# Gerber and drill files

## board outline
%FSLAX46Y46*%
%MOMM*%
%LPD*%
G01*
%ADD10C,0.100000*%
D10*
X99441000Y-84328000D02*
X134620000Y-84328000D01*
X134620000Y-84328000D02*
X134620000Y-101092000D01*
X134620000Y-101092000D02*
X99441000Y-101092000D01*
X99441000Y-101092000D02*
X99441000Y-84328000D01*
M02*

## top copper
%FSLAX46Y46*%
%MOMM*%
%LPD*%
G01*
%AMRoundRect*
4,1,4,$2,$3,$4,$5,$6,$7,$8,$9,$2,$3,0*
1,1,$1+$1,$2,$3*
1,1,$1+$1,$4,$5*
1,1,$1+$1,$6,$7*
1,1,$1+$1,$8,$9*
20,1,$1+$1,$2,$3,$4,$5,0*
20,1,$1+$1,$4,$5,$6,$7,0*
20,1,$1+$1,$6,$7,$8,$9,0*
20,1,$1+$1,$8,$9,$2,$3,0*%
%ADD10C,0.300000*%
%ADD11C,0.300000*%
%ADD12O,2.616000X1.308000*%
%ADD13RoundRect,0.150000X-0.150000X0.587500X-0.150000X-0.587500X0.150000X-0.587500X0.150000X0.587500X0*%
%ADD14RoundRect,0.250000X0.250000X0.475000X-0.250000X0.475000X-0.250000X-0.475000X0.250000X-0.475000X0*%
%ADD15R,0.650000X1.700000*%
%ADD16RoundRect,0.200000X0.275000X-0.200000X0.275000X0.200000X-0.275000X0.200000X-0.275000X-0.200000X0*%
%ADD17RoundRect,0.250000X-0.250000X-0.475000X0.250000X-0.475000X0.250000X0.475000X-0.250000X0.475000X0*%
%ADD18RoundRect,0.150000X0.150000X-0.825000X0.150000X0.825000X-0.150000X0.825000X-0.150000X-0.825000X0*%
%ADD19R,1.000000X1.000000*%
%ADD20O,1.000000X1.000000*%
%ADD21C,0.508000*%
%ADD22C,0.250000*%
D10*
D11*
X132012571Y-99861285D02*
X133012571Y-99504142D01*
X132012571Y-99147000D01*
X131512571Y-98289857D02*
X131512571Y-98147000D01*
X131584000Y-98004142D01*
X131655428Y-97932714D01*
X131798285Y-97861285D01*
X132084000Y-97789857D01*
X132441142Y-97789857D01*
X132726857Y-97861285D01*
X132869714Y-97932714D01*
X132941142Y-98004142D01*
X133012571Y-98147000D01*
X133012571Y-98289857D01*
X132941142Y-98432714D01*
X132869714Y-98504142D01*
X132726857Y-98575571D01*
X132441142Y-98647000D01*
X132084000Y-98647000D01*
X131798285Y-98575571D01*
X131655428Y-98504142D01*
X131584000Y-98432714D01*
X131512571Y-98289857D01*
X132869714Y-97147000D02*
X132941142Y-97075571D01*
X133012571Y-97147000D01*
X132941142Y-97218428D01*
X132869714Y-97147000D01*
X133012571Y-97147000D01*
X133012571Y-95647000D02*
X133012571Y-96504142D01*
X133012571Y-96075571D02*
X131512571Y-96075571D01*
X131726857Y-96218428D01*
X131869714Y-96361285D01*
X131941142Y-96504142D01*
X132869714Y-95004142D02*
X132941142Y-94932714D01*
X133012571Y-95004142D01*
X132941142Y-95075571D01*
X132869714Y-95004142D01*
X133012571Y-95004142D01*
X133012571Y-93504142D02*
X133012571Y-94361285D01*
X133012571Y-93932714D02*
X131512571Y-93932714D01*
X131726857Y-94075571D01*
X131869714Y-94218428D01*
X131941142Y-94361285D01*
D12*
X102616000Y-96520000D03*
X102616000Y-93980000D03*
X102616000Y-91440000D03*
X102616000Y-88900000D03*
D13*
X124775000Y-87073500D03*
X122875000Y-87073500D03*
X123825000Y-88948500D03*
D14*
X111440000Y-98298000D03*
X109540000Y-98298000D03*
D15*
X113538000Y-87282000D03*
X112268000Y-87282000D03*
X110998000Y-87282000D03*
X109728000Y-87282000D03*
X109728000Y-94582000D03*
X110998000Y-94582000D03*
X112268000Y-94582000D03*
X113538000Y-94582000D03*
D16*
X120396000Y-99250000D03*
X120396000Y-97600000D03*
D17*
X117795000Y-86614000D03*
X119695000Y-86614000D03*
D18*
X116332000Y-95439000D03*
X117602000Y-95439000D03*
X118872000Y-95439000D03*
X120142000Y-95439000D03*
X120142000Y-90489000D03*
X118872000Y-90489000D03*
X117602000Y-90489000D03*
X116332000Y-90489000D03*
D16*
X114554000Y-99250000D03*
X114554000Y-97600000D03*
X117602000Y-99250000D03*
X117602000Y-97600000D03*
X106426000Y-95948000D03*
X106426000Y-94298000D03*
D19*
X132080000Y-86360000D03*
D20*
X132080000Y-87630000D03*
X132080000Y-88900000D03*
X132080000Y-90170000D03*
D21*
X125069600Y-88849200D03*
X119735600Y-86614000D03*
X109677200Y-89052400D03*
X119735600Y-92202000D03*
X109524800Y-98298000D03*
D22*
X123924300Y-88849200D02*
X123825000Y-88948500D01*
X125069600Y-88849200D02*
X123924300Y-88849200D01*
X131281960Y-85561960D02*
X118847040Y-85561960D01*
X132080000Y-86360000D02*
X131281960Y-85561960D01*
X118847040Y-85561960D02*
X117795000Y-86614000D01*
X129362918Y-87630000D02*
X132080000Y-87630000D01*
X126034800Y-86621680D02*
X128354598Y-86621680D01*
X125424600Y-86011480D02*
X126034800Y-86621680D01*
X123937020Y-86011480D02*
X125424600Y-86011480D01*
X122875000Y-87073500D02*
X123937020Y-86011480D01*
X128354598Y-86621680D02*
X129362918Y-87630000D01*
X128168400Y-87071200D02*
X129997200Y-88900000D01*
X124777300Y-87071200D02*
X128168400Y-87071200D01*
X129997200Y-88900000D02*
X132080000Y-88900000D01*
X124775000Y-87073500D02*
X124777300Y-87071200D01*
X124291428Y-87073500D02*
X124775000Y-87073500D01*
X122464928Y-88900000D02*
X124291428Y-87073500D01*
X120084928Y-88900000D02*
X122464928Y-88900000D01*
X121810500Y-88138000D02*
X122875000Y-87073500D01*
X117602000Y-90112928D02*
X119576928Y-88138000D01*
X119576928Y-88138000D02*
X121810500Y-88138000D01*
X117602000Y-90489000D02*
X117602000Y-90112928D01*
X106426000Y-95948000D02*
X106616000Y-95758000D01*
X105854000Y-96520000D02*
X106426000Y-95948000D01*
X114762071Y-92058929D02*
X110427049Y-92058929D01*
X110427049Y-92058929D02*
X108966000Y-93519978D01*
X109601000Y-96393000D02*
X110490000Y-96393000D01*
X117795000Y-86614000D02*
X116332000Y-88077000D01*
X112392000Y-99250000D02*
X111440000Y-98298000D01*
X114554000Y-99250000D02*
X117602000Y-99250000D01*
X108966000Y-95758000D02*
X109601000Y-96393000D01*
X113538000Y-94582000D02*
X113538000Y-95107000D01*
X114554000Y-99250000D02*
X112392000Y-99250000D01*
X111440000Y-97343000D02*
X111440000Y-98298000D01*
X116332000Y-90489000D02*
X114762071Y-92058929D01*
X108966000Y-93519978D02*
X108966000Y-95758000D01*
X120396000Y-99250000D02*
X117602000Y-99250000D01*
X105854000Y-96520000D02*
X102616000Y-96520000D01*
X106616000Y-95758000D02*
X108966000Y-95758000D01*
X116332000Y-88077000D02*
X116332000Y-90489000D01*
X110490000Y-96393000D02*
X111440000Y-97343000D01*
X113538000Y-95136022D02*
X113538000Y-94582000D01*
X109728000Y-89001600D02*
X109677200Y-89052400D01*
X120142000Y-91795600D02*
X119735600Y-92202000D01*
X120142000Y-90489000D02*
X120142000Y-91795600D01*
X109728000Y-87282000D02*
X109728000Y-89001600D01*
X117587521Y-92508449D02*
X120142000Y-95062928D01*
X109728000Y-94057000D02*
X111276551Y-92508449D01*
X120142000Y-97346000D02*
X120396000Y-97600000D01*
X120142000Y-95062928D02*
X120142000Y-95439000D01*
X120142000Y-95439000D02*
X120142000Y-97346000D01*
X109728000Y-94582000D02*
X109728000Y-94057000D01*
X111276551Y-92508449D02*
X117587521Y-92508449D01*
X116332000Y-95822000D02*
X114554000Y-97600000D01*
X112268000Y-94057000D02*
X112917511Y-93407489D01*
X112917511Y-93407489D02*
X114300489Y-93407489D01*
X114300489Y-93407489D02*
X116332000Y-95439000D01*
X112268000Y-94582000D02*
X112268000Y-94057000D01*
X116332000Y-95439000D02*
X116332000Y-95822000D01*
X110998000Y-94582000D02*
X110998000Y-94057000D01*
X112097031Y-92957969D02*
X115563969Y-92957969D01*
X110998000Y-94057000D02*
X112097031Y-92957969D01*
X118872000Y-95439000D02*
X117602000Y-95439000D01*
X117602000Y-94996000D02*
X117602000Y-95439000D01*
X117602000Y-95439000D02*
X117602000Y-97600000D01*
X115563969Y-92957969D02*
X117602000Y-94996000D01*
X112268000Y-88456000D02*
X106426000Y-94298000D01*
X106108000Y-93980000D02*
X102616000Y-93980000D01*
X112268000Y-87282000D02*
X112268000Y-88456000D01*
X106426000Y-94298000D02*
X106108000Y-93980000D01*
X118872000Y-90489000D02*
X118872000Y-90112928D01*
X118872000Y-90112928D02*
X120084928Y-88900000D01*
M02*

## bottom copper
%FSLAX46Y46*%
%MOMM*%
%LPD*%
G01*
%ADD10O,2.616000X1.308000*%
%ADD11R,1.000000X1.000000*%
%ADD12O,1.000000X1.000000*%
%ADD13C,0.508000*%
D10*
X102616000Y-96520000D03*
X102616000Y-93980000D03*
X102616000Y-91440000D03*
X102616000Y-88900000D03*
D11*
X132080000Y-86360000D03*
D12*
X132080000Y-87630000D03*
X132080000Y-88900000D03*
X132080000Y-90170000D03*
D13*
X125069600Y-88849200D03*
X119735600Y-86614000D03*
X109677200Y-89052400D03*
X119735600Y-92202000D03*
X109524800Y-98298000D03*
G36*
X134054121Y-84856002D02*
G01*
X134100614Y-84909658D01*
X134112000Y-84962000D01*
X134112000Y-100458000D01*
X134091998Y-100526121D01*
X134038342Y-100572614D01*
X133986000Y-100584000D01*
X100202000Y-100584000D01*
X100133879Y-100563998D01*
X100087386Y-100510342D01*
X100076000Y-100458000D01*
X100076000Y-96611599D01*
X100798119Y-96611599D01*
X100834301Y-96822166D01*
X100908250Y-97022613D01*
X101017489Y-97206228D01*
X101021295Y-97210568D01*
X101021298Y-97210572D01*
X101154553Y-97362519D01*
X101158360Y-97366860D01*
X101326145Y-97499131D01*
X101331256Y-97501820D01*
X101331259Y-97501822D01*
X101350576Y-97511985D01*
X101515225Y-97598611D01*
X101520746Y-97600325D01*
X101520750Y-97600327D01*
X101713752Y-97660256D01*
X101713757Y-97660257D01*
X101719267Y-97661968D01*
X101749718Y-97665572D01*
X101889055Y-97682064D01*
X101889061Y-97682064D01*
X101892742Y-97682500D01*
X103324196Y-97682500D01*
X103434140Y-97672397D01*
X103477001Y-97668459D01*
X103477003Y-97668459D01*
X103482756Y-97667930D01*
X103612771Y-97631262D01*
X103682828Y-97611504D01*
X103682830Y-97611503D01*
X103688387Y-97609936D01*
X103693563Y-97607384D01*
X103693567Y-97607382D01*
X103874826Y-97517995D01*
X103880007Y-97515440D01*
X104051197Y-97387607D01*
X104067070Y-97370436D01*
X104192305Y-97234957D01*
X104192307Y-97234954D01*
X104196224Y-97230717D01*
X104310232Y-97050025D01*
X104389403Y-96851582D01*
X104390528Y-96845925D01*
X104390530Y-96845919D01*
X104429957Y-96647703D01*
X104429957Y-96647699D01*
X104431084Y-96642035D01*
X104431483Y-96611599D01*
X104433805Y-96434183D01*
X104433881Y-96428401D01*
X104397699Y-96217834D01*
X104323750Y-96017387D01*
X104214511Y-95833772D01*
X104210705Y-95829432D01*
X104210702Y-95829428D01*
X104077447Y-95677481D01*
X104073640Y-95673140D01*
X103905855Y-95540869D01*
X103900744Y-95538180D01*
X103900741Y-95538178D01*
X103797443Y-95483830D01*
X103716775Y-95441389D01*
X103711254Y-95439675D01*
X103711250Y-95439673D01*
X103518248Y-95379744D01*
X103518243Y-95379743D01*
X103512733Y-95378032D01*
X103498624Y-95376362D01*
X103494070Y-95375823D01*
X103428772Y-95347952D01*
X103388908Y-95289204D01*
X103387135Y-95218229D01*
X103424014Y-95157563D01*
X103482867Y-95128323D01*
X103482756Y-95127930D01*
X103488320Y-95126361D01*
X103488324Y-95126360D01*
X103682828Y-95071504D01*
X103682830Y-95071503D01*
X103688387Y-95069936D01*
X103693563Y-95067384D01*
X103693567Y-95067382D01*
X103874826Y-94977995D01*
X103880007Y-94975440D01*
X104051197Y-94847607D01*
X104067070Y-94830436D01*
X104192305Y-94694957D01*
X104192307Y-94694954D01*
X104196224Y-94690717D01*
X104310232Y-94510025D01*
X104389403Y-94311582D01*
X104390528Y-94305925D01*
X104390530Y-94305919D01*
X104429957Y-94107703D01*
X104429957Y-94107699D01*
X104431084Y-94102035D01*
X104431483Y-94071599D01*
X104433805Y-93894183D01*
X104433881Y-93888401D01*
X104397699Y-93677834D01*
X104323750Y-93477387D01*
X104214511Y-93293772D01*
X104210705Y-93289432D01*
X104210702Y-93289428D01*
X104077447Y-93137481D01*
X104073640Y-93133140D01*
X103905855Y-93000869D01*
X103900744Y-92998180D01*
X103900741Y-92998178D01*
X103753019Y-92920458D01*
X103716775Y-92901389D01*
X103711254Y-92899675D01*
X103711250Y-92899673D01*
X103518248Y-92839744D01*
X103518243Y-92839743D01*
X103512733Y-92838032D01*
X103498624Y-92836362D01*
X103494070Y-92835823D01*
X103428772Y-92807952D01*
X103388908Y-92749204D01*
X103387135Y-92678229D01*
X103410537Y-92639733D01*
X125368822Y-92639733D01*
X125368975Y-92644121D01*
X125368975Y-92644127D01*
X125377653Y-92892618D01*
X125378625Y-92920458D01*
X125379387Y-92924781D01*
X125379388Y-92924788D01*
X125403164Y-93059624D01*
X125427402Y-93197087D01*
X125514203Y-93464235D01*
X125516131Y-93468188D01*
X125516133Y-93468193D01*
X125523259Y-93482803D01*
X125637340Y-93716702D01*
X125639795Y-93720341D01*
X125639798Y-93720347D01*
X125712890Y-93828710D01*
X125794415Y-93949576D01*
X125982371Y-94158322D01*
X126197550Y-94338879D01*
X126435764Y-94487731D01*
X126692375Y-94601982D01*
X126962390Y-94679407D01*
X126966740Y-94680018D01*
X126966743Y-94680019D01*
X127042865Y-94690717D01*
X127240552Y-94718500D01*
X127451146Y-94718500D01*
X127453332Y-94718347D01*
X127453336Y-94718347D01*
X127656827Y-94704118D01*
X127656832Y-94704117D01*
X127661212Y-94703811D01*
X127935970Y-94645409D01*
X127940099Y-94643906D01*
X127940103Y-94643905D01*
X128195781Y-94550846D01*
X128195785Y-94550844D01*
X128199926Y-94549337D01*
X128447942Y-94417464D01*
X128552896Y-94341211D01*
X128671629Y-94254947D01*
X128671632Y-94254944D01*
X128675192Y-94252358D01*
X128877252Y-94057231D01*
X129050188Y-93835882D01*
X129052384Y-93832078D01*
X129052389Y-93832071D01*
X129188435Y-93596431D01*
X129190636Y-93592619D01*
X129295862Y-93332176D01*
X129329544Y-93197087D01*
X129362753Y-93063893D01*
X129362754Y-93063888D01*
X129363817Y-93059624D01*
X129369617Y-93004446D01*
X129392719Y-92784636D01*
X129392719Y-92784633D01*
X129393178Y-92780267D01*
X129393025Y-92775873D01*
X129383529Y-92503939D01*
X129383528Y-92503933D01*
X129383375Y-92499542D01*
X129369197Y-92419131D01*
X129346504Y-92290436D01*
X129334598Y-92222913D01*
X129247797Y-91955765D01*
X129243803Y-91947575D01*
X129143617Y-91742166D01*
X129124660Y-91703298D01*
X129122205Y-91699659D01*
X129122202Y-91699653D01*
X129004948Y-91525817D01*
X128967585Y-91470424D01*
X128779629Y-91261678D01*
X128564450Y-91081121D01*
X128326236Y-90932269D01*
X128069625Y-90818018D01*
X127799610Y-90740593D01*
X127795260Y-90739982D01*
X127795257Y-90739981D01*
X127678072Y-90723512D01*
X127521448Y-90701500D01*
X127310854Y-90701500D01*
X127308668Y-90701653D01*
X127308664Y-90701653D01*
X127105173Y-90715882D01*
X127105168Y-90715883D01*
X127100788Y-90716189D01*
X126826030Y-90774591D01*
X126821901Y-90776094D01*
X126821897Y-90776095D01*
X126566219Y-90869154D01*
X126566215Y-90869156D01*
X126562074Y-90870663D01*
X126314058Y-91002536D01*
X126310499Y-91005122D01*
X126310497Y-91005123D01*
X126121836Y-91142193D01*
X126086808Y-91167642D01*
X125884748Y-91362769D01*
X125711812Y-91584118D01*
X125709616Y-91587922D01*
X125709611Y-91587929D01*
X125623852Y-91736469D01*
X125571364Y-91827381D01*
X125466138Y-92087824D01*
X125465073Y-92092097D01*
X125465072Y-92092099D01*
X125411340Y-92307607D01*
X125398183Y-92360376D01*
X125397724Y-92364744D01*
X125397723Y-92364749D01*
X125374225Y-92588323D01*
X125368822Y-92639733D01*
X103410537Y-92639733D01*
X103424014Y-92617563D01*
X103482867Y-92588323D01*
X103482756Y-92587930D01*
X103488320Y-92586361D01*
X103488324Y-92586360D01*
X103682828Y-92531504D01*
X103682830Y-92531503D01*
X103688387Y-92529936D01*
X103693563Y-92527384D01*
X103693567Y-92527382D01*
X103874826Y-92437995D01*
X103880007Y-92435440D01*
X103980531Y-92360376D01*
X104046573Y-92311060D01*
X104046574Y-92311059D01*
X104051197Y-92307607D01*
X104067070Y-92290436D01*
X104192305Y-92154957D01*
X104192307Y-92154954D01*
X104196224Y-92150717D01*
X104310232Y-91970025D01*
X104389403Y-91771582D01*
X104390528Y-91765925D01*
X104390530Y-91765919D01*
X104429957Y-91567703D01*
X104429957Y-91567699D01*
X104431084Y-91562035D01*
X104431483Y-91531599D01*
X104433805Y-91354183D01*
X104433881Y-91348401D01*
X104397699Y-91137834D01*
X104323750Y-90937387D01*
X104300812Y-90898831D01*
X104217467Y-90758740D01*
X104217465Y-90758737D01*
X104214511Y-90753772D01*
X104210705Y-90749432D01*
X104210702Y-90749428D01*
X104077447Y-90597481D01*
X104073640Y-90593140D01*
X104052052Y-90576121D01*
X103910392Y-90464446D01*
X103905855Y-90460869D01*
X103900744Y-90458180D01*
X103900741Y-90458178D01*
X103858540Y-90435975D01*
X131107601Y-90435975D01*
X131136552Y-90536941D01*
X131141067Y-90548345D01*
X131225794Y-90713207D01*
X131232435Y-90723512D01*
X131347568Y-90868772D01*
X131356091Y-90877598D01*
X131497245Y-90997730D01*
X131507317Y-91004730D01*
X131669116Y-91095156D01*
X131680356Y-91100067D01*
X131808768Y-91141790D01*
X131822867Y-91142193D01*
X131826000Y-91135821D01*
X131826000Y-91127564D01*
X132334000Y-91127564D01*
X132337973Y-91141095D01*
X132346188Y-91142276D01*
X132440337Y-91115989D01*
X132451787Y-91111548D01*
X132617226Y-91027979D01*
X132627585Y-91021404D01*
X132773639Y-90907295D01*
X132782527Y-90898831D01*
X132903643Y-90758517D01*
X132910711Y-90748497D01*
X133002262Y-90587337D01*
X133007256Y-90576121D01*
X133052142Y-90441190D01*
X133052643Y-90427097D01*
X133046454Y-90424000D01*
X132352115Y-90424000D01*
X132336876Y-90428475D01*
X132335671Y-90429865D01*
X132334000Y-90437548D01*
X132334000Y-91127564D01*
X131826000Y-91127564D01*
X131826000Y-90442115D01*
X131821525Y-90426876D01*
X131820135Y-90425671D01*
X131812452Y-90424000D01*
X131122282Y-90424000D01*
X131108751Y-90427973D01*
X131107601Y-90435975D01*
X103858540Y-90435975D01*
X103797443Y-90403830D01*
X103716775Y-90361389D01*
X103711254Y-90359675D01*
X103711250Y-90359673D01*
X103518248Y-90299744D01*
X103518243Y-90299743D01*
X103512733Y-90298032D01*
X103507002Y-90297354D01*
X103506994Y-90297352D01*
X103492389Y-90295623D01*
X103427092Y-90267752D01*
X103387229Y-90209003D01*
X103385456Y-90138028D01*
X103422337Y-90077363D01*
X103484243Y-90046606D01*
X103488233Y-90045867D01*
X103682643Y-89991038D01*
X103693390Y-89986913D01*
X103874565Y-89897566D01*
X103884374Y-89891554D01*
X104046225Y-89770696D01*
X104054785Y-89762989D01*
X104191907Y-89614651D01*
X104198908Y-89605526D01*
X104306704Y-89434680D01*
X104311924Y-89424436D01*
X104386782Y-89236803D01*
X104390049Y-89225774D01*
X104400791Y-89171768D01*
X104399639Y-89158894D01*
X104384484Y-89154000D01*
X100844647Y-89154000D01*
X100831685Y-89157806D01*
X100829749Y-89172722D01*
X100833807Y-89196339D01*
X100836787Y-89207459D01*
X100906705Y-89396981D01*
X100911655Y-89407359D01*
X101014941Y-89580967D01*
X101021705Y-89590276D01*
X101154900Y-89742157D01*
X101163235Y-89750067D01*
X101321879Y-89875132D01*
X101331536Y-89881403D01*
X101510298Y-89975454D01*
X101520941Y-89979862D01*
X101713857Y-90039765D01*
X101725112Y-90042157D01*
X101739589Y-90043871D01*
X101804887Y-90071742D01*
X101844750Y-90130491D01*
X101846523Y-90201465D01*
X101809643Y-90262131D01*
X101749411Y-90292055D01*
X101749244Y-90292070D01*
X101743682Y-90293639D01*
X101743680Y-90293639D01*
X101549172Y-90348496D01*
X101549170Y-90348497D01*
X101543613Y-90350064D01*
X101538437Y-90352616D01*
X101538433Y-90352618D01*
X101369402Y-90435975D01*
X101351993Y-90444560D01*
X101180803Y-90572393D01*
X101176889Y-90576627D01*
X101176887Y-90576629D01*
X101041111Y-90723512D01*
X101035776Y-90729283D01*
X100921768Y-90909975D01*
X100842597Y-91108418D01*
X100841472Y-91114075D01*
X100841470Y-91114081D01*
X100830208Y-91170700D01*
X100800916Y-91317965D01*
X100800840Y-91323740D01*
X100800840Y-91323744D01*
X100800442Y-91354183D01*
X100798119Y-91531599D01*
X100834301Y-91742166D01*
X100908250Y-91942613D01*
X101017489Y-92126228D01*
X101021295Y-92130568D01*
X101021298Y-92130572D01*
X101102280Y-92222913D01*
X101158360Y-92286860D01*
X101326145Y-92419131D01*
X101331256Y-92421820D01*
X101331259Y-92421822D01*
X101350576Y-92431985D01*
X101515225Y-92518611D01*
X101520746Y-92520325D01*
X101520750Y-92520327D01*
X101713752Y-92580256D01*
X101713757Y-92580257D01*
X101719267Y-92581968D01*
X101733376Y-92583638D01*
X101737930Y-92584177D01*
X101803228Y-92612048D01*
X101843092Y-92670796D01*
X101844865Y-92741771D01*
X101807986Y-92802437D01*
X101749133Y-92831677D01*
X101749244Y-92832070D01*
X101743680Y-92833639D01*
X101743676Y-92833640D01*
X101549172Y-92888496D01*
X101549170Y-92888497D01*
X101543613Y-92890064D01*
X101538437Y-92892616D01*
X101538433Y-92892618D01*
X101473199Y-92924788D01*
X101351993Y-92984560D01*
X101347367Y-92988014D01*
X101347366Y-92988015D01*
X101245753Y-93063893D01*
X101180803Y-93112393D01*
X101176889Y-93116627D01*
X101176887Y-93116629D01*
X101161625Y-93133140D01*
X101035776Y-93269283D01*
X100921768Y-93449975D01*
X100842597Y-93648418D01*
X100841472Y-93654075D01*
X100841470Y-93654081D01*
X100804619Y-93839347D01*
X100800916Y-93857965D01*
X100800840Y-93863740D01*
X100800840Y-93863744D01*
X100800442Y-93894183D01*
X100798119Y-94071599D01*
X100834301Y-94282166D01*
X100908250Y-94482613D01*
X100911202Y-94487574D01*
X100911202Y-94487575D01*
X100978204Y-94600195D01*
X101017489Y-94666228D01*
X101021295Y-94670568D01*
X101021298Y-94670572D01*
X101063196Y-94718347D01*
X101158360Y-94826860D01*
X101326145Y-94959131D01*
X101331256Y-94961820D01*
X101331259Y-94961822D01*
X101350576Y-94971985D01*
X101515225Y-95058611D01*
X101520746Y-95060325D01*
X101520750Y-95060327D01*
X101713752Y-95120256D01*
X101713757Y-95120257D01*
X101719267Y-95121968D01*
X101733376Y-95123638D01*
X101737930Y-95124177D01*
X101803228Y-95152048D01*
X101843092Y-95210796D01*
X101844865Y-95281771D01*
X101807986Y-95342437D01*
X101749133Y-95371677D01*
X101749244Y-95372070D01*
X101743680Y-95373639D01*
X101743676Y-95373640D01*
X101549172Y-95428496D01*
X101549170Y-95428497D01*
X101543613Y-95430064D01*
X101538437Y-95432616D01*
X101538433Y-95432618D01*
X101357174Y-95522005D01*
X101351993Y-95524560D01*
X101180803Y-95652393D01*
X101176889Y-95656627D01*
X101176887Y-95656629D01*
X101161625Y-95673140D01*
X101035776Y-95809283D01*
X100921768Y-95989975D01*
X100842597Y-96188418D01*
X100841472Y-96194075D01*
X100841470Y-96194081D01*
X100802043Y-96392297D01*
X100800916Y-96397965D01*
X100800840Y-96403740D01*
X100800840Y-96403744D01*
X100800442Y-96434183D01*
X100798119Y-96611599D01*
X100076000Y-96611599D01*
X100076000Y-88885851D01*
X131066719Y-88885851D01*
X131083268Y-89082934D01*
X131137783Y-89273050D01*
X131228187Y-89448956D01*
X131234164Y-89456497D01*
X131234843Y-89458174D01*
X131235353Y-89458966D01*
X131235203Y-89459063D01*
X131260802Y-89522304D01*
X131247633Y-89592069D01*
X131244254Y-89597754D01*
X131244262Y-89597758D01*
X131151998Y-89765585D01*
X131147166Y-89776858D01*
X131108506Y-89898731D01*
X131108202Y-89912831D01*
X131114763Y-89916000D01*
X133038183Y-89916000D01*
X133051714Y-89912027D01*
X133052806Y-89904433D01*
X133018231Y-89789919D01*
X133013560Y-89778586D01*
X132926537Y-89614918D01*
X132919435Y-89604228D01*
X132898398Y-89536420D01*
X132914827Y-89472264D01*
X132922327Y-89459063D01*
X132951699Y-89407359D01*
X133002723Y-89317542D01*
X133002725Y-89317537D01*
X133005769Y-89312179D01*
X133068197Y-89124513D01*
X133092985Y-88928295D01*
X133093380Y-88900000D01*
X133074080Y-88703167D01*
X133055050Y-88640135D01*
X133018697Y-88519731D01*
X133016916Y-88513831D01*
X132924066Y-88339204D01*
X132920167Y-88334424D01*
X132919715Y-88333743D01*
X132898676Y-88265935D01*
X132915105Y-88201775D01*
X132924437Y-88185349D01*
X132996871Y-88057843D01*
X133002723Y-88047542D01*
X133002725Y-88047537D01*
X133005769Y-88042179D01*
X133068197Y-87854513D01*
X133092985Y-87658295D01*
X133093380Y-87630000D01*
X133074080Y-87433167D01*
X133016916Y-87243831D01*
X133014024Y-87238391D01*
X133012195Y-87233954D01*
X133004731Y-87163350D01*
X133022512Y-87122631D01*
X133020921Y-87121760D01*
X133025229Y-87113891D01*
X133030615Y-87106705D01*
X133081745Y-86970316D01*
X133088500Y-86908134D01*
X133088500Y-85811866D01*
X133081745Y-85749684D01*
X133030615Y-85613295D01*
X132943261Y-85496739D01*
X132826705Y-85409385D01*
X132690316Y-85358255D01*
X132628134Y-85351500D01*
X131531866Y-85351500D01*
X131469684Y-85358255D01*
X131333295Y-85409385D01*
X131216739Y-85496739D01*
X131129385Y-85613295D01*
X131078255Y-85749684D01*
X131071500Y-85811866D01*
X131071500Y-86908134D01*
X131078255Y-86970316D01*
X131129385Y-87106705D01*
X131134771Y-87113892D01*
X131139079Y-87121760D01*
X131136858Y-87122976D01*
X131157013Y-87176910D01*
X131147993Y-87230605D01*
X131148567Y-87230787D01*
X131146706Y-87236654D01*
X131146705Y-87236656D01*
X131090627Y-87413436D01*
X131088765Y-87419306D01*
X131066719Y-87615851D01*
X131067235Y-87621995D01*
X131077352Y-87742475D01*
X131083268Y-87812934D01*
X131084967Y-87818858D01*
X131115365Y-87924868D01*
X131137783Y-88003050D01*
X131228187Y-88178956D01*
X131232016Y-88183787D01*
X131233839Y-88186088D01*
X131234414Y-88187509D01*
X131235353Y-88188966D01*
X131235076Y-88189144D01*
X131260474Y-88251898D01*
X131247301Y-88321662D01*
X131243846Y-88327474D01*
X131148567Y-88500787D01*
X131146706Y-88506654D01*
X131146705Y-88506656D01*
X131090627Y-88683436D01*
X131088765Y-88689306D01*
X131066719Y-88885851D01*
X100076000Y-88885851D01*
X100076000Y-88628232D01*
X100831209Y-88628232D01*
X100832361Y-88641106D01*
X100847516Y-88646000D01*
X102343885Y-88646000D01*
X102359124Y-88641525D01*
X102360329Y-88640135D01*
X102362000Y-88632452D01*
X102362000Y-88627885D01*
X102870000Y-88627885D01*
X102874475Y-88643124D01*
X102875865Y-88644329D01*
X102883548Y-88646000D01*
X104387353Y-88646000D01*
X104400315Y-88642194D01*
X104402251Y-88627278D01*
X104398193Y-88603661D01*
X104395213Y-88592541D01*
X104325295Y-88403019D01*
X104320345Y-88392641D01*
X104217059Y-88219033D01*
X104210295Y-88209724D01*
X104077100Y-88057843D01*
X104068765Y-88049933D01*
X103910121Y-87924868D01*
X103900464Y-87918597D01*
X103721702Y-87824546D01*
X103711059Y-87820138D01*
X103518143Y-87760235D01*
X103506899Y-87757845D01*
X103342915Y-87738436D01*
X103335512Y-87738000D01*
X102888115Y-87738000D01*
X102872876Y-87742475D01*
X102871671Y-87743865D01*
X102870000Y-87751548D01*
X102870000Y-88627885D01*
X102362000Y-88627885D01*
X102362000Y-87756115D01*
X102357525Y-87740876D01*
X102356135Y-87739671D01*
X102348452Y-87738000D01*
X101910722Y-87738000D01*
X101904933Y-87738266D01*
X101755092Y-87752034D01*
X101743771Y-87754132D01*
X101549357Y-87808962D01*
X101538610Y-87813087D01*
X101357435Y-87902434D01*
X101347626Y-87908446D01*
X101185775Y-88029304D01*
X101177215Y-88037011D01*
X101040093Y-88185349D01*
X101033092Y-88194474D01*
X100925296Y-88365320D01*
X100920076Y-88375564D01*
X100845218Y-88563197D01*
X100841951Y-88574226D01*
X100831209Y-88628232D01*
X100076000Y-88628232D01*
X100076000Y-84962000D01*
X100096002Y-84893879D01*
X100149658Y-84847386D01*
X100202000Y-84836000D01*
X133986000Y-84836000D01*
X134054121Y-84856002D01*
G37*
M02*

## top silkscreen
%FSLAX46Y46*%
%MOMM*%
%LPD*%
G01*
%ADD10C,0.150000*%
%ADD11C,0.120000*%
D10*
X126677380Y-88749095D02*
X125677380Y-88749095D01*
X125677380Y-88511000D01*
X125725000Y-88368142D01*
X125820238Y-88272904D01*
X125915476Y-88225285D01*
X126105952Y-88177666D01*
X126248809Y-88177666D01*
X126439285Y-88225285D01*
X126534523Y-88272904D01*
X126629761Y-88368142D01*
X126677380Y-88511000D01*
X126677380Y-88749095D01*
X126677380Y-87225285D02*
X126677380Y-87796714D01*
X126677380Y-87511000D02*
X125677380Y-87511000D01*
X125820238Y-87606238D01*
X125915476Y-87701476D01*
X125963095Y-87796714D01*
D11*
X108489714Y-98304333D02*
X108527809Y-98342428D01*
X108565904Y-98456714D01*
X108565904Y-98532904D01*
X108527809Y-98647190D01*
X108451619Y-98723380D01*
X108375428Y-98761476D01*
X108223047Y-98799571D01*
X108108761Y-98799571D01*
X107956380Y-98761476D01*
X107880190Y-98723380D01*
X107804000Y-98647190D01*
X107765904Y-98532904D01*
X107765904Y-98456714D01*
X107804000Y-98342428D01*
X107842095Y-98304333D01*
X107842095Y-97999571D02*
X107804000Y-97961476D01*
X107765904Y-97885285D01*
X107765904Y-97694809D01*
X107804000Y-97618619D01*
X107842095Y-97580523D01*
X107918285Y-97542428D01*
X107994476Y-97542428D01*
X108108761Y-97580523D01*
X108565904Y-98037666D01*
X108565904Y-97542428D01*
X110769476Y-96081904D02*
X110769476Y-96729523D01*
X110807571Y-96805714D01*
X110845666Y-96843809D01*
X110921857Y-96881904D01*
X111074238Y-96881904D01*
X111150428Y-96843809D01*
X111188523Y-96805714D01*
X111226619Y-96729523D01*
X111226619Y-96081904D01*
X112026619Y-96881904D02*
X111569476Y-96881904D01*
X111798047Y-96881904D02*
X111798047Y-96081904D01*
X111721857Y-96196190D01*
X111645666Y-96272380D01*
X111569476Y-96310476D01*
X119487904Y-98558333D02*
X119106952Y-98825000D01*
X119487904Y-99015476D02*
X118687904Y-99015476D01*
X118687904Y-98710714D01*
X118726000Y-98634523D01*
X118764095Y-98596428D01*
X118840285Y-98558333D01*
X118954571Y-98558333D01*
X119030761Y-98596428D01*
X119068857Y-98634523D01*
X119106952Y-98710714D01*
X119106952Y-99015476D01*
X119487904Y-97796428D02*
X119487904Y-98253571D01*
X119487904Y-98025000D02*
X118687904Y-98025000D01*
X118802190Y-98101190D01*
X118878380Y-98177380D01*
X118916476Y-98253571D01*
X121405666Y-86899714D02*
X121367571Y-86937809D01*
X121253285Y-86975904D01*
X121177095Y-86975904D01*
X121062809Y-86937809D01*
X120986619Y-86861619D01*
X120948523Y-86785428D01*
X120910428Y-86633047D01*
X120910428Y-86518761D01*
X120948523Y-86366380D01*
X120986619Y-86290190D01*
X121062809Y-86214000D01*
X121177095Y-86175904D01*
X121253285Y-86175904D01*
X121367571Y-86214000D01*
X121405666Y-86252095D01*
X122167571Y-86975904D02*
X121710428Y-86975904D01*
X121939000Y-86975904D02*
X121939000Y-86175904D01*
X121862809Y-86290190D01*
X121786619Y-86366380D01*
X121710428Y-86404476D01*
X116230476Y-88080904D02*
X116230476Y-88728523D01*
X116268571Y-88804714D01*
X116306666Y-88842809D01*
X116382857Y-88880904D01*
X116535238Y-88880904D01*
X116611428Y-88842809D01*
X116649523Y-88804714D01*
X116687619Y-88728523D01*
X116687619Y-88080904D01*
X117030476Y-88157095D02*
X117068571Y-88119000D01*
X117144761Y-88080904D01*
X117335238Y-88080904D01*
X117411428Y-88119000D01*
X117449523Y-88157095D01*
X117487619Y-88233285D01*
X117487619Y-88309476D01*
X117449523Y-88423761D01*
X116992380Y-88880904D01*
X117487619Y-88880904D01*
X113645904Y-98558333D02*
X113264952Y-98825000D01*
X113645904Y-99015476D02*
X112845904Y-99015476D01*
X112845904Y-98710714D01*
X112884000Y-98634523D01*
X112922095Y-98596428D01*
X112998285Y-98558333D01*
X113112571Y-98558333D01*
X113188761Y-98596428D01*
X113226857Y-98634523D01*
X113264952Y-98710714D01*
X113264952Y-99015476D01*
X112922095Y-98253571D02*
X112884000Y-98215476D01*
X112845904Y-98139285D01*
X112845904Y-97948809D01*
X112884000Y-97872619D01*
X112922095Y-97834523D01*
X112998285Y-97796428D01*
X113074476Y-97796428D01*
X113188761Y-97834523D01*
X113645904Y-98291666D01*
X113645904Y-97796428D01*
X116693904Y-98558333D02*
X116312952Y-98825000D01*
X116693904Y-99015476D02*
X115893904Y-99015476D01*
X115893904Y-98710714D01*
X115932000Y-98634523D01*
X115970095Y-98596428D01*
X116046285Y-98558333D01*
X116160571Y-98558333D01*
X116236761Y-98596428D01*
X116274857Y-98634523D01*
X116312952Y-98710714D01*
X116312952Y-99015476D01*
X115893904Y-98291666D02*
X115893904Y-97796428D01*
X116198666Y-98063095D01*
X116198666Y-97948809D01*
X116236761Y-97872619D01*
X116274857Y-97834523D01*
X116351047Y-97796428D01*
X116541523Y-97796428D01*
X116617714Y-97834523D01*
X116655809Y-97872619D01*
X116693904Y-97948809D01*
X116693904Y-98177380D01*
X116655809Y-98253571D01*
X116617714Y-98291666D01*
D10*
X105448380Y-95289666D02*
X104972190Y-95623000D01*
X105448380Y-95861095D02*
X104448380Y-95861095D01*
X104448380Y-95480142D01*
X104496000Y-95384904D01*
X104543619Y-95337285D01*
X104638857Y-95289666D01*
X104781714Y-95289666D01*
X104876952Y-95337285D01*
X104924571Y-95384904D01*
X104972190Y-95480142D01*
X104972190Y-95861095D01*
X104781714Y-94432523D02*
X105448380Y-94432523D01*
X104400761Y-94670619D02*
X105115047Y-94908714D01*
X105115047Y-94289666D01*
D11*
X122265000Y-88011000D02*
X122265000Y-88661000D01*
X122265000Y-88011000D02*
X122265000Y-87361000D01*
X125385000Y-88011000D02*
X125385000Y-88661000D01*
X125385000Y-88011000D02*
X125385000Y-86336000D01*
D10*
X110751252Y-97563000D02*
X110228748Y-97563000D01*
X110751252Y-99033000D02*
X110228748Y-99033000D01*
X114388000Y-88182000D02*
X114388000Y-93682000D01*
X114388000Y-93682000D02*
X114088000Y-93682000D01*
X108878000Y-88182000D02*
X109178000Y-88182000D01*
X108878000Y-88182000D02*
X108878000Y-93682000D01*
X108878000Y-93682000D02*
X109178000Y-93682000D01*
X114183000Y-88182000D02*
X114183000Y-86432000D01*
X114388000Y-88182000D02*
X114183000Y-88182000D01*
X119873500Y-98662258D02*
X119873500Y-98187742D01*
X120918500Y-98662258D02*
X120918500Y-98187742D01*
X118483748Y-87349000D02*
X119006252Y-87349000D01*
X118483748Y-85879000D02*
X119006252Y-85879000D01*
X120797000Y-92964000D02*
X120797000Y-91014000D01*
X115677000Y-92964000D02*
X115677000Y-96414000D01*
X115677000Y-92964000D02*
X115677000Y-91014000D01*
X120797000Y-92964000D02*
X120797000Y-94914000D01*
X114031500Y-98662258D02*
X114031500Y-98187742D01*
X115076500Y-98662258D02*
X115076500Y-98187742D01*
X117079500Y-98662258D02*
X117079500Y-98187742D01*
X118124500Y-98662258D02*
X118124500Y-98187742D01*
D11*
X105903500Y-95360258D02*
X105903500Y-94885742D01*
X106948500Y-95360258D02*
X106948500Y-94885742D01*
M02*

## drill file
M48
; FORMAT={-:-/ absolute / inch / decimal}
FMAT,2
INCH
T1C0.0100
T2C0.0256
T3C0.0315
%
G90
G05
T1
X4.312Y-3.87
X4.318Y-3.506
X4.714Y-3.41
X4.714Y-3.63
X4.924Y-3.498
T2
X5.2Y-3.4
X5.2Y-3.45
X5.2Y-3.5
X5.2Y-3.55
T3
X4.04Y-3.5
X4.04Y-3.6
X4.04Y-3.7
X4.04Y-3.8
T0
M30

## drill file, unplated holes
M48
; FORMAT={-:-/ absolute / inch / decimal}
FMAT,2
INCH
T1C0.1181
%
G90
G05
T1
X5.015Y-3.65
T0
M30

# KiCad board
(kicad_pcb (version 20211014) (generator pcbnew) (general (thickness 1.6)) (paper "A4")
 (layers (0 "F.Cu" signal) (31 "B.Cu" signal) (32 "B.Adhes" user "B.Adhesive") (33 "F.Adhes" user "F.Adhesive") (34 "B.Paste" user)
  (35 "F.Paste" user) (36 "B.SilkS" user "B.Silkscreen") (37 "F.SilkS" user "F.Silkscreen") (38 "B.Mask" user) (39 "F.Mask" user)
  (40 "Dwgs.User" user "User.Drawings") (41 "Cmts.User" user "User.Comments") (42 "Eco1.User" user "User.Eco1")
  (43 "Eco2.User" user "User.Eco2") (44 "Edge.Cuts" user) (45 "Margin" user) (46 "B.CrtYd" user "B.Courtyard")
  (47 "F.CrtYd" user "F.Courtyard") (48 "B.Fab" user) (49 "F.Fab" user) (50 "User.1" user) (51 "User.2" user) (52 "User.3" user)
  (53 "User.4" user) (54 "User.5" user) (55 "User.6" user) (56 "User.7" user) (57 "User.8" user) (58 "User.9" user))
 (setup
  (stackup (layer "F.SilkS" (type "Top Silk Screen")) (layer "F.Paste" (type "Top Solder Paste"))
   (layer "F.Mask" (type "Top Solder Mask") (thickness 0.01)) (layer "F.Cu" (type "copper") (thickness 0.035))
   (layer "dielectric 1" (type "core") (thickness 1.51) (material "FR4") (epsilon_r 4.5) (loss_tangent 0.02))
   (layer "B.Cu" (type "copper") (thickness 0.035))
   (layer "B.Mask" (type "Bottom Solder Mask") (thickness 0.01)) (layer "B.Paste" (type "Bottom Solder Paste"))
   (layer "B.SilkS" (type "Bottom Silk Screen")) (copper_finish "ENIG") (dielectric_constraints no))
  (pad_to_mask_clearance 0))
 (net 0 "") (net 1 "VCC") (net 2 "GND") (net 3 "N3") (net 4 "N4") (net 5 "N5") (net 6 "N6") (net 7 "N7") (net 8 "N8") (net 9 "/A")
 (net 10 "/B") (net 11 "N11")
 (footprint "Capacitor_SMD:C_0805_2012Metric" (layer "F.Cu") (at 110.49 98.298 180)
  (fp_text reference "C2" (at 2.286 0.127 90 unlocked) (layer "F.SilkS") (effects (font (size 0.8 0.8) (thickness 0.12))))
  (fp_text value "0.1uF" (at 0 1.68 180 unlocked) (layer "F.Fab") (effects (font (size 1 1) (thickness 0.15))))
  (fp_line (start -0.261252 0.735) (end 0.261252 0.735) (layer "F.SilkS") (width 0.15))
  (fp_line (start -0.261252 -0.735) (end 0.261252 -0.735) (layer "F.SilkS") (width 0.15))
  (pad "1" smd roundrect locked (at -0.95 0 180) (size 1 1.45) (layers "F.Cu" "F.Paste" "F.Mask") (roundrect_rratio 0.25) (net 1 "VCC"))
  (pad "2" smd roundrect locked (at 0.95 0 180) (size 1 1.45) (layers "F.Cu" "F.Paste" "F.Mask") (roundrect_rratio 0.25) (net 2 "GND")))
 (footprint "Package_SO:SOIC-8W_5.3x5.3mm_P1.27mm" (layer "F.Cu") (at 111.633 90.932 -90)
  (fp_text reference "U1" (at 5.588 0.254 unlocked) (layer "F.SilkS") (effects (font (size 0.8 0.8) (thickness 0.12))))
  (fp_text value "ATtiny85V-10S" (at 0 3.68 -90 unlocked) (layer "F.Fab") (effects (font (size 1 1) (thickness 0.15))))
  (fp_line (start -2.75 -2.755) (end 2.75 -2.755) (layer "F.SilkS") (width 0.15))
  (fp_line (start 2.75 -2.755) (end 2.75 -2.455) (layer "F.SilkS") (width 0.15))
  (fp_line (start -2.75 2.755) (end -2.75 2.455) (layer "F.SilkS") (width 0.15))
  (fp_line (start -2.75 2.755) (end 2.75 2.755) (layer "F.SilkS") (width 0.15))
  (fp_line (start 2.75 2.755) (end 2.75 2.455) (layer "F.SilkS") (width 0.15))
  (fp_line (start -2.75 -2.55) (end -4.5 -2.55) (layer "F.SilkS") (width 0.15))
  (fp_line (start -2.75 -2.755) (end -2.75 -2.55) (layer "F.SilkS") (width 0.15))
  (pad "1" smd rect locked (at -3.65 -1.905 270) (size 1.7 0.65) (layers "F.Cu" "F.Paste" "F.Mask") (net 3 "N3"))
  (pad "2" smd rect locked (at -3.65 -0.635 270) (size 1.7 0.65) (layers "F.Cu" "F.Paste" "F.Mask") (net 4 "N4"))
  (pad "3" smd rect locked (at -3.65 0.635 270) (size 1.7 0.65) (layers "F.Cu" "F.Paste" "F.Mask") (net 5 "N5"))
  (pad "4" smd rect locked (at -3.65 1.905 270) (size 1.7 0.65) (layers "F.Cu" "F.Paste" "F.Mask") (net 2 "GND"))
  (pad "5" smd rect locked (at 3.65 1.905 270) (size 1.7 0.65) (layers "F.Cu" "F.Paste" "F.Mask") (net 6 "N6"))
  (pad "6" smd rect locked (at 3.65 0.635 270) (size 1.7 0.65) (layers "F.Cu" "F.Paste" "F.Mask") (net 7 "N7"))
  (pad "7" smd rect locked (at 3.65 -0.635 270) (size 1.7 0.65) (layers "F.Cu" "F.Paste" "F.Mask") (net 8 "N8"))
  (pad "8" smd rect locked (at 3.65 -1.905 270) (size 1.7 0.65) (layers "F.Cu" "F.Paste" "F.Mask") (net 1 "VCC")))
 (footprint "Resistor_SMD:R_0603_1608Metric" (layer "F.Cu") (at 120.396 98.425 90)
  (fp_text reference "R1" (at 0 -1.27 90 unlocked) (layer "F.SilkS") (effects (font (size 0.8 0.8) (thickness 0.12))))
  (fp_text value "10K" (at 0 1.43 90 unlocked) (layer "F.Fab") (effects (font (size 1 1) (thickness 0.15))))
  (fp_line (start -0.237258 -0.5225) (end 0.237258 -0.5225) (layer "F.SilkS") (width 0.15))
  (fp_line (start -0.237258 0.5225) (end 0.237258 0.5225) (layer "F.SilkS") (width 0.15))
  (pad "1" smd roundrect locked (at -0.825 0 90) (size 0.8 0.95) (layers "F.Cu" "F.Paste" "F.Mask") (roundrect_rratio 0.25) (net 1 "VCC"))
  (pad "2" smd roundrect locked (at 0.825 0 90) (size 0.8 0.95) (layers "F.Cu" "F.Paste" "F.Mask") (roundrect_rratio 0.25) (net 6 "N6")))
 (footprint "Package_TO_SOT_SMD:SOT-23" (layer "F.Cu") (at 123.825 88.011 -90)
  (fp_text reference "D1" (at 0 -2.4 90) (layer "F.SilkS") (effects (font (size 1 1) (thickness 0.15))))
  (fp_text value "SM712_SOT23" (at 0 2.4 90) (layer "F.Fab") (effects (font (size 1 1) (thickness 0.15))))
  (fp_line (start 0 -1.56) (end -1.675 -1.56) (layer "F.SilkS") (width 0.12))
  (fp_line (start 0 1.56) (end 0.65 1.56) (layer "F.SilkS") (width 0.12))
  (fp_line (start 0 -1.56) (end 0.65 -1.56) (layer "F.SilkS") (width 0.12))
  (fp_line (start 0 1.56) (end -0.65 1.56) (layer "F.SilkS") (width 0.12))
  (pad "1" smd roundrect locked (at -0.9375 -0.95 270) (size 1.475 0.6) (layers "F.Cu" "F.Paste" "F.Mask") (roundrect_rratio 0.25)
   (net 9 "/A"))
  (pad "2" smd roundrect locked (at -0.9375 0.95 270) (size 1.475 0.6) (layers "F.Cu" "F.Paste" "F.Mask") (roundrect_rratio 0.25)
   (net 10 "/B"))
  (pad "3" smd roundrect locked (at 0.9375 0 270) (size 1.475 0.6) (layers "F.Cu" "F.Paste" "F.Mask") (roundrect_rratio 0.25) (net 2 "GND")))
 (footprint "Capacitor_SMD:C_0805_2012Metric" (layer "F.Cu") (at 118.745 86.614)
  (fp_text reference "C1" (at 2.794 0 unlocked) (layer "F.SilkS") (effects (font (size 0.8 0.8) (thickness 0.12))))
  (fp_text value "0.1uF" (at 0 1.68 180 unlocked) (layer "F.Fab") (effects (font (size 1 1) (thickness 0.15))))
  (fp_line (start -0.261252 0.735) (end 0.261252 0.735) (layer "F.SilkS") (width 0.15))
  (fp_line (start -0.261252 -0.735) (end 0.261252 -0.735) (layer "F.SilkS") (width 0.15))
  (pad "1" smd roundrect locked (at -0.95 0) (size 1 1.45) (layers "F.Cu" "F.Paste" "F.Mask") (roundrect_rratio 0.25) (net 1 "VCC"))
  (pad "2" smd roundrect locked (at 0.95 0) (size 1 1.45) (layers "F.Cu" "F.Paste" "F.Mask") (roundrect_rratio 0.25) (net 2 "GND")))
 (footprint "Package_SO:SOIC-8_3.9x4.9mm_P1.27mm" (layer "F.Cu") (at 118.237 92.964 90)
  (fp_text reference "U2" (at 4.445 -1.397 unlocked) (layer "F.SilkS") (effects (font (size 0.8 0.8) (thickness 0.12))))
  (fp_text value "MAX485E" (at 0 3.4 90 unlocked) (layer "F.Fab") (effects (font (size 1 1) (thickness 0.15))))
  (fp_line (start 0 2.56) (end 1.95 2.56) (layer "F.SilkS") (width 0.15))
  (fp_line (start 0 -2.56) (end -3.45 -2.56) (layer "F.SilkS") (width 0.15))
  (fp_line (start 0 -2.56) (end 1.95 -2.56) (layer "F.SilkS") (width 0.15))
  (fp_line (start 0 2.56) (end -1.95 2.56) (layer "F.SilkS") (width 0.15))
  (pad "1" smd roundrect locked (at -2.475 -1.905 90) (size 1.95 0.6) (layers "F.Cu" "F.Paste" "F.Mask") (roundrect_rratio 0.25)
   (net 8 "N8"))
  (pad "2" smd roundrect locked (at -2.475 -0.635 90) (size 1.95 0.6) (layers "F.Cu" "F.Paste" "F.Mask") (roundrect_rratio 0.25)
   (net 7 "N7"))
  (pad "3" smd roundrect locked (at -2.475 0.635 90) (size 1.95 0.6) (layers "F.Cu" "F.Paste" "F.Mask") (roundrect_rratio 0.25) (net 7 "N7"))
  (pad "4" smd roundrect locked (at -2.475 1.905 90) (size 1.95 0.6) (layers "F.Cu" "F.Paste" "F.Mask") (roundrect_rratio 0.25) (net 6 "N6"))
  (pad "5" smd roundrect locked (at 2.475 1.905 90) (size 1.95 0.6) (layers "F.Cu" "F.Paste" "F.Mask") (roundrect_rratio 0.25) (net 2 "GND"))
  (pad "6" smd roundrect locked (at 2.475 0.635 90) (size 1.95 0.6) (layers "F.Cu" "F.Paste" "F.Mask") (roundrect_rratio 0.25) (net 9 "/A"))
  (pad "7" smd roundrect locked (at 2.475 -0.635 90) (size 1.95 0.6) (layers "F.Cu" "F.Paste" "F.Mask") (roundrect_rratio 0.25)
   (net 10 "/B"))
  (pad "8" smd roundrect locked (at 2.475 -1.905 90) (size 1.95 0.6) (layers "F.Cu" "F.Paste" "F.Mask") (roundrect_rratio 0.25)
   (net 1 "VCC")))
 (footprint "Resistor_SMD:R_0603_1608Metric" (layer "F.Cu") (at 114.554 98.425 90)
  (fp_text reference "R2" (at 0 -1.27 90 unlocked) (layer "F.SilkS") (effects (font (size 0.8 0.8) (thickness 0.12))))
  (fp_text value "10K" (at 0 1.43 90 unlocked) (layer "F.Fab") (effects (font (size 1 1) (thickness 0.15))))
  (fp_line (start -0.237258 -0.5225) (end 0.237258 -0.5225) (layer "F.SilkS") (width 0.15))
  (fp_line (start -0.237258 0.5225) (end 0.237258 0.5225) (layer "F.SilkS") (width 0.15))
  (pad "1" smd roundrect locked (at -0.825 0 90) (size 0.8 0.95) (layers "F.Cu" "F.Paste" "F.Mask") (roundrect_rratio 0.25) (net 1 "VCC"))
  (pad "2" smd roundrect locked (at 0.825 0 90) (size 0.8 0.95) (layers "F.Cu" "F.Paste" "F.Mask") (roundrect_rratio 0.25) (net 8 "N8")))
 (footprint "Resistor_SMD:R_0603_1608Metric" (layer "F.Cu") (at 117.602 98.425 90)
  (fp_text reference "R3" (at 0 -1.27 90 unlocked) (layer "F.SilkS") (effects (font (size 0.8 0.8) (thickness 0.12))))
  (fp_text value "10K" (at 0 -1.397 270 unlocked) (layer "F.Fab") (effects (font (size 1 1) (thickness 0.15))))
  (fp_line (start -0.237258 -0.5225) (end 0.237258 -0.5225) (layer "F.SilkS") (width 0.15))
  (fp_line (start -0.237258 0.5225) (end 0.237258 0.5225) (layer "F.SilkS") (width 0.15))
  (pad "1" smd roundrect locked (at -0.825 0 90) (size 0.8 0.95) (layers "F.Cu" "F.Paste" "F.Mask") (roundrect_rratio 0.25) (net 1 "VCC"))
  (pad "2" smd roundrect locked (at 0.825 0 90) (size 0.8 0.95) (layers "F.Cu" "F.Paste" "F.Mask") (roundrect_rratio 0.25) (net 7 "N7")))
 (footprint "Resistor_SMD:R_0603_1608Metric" (layer "F.Cu") (at 106.426 95.123 90)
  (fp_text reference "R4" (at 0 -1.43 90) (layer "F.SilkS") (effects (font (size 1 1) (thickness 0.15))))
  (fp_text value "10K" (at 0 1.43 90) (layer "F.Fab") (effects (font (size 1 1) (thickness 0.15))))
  (fp_line (start -0.237258 -0.5225) (end 0.237258 -0.5225) (layer "F.SilkS") (width 0.12))
  (fp_line (start -0.237258 0.5225) (end 0.237258 0.5225) (layer "F.SilkS") (width 0.12))
  (pad "1" smd roundrect locked (at -0.825 0 90) (size 0.8 0.95) (layers "F.Cu" "F.Paste" "F.Mask") (roundrect_rratio 0.25) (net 1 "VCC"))
  (pad "2" smd roundrect locked (at 0.825 0 90) (size 0.8 0.95) (layers "F.Cu" "F.Paste" "F.Mask") (roundrect_rratio 0.25) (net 4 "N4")))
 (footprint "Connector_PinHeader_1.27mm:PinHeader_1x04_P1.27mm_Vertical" (layer "B.Cu") (at 132.08 86.36 180)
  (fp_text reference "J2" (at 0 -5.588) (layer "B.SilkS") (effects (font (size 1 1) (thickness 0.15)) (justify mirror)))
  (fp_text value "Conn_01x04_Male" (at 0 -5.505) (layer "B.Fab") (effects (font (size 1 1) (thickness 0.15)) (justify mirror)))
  (pad "1" thru_hole rect locked (at 0 0 180) (size 1 1) (drill 0.65) (layers *.Cu *.Mask) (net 1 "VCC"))
  (pad "2" thru_hole oval locked (at 0 -1.27 180) (size 1 1) (drill 0.65) (layers *.Cu *.Mask) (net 10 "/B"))
  (pad "3" thru_hole oval locked (at 0 -2.54 180) (size 1 1) (drill 0.65) (layers *.Cu *.Mask) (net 9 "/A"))
  (pad "4" thru_hole oval locked (at 0 -3.81 180) (size 1 1) (drill 0.65) (layers *.Cu *.Mask) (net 2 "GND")))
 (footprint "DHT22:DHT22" (layer "B.Cu") (at 102.616 92.71 90)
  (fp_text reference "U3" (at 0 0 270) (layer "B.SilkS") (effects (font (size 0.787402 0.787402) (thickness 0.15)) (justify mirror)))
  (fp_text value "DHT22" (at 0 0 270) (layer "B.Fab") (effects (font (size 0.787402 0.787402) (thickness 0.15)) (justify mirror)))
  (pad "" np_thru_hole circle locked (at 0 24.765 90) (size 3 3) (drill 3) (layers *.Cu *.Mask))
  (pad "DATA" thru_hole oval locked (at -1.27 0 90) (size 1.308 2.616) (drill 0.8) (layers *.Cu *.Mask) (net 4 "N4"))
  (pad "GND" thru_hole oval locked (at 3.81 0 90) (size 1.308 2.616) (drill 0.8) (layers *.Cu *.Mask) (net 2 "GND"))
  (pad "NC" thru_hole oval locked (at 1.27 0 90) (size 1.308 2.616) (drill 0.8) (layers *.Cu *.Mask) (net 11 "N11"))
  (pad "VDD" thru_hole oval locked (at -3.81 0 90) (size 1.308 2.616) (drill 0.8) (layers *.Cu *.Mask) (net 1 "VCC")))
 (gr_rect (start 99.441 84.328) (end 134.62 101.092) (layer "Edge.Cuts") (width 0.1) (fill none))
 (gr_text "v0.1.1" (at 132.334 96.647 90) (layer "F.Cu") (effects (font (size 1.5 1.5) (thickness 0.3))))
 (segment (start 106.426 95.948) (end 106.616 95.758) (width 0.25) (layer "F.Cu") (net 1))
 (segment (start 105.854 96.52) (end 106.426 95.948) (width 0.25) (layer "F.Cu") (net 1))
 (segment (start 114.762071 92.058929) (end 110.427049 92.058929) (width 0.25) (layer "F.Cu") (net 1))
 (segment (start 110.427049 92.058929) (end 108.966 93.519978) (width 0.25) (layer "F.Cu") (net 1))
 (segment (start 109.601 96.393) (end 110.49 96.393) (width 0.25) (layer "F.Cu") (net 1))
 (segment (start 117.795 86.614) (end 116.332 88.077) (width 0.25) (layer "F.Cu") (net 1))
 (segment (start 131.28196 85.56196) (end 118.84704 85.56196) (width 0.25) (layer "F.Cu") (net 1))
 (segment (start 112.392 99.25) (end 111.44 98.298) (width 0.25) (layer "F.Cu") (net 1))
 (segment (start 114.554 99.25) (end 117.602 99.25) (width 0.25) (layer "F.Cu") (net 1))
 (segment (start 108.966 95.758) (end 109.601 96.393) (width 0.25) (layer "F.Cu") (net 1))
 (segment (start 113.538 94.582) (end 113.538 95.107) (width 0.25) (layer "F.Cu") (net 1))
 (segment (start 114.554 99.25) (end 112.392 99.25) (width 0.25) (layer "F.Cu") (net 1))
 (segment (start 111.44 97.343) (end 111.44 98.298) (width 0.25) (layer "F.Cu") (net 1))
 (segment (start 116.332 90.489) (end 114.762071 92.058929) (width 0.25) (layer "F.Cu") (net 1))
 (segment (start 108.966 93.519978) (end 108.966 95.758) (width 0.25) (layer "F.Cu") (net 1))
 (segment (start 120.396 99.25) (end 117.602 99.25) (width 0.25) (layer "F.Cu") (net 1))
 (segment (start 105.854 96.52) (end 102.616 96.52) (width 0.25) (layer "F.Cu") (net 1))
 (segment (start 106.616 95.758) (end 108.966 95.758) (width 0.25) (layer "F.Cu") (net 1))
 (segment (start 118.84704 85.56196) (end 117.795 86.614) (width 0.25) (layer "F.Cu") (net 1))
 (segment (start 116.332 88.077) (end 116.332 90.489) (width 0.25) (layer "F.Cu") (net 1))
 (segment (start 110.49 96.393) (end 111.44 97.343) (width 0.25) (layer "F.Cu") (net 1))
 (segment (start 113.538 95.136022) (end 113.538 94.582) (width 0.25) (layer "F.Cu") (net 1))
 (segment (start 132.08 86.36) (end 131.28196 85.56196) (width 0.25) (layer "F.Cu") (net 1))
 (segment (start 109.728 89.0016) (end 109.6772 89.0524) (width 0.25) (layer "F.Cu") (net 2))
 (segment (start 123.9243 88.8492) (end 123.825 88.9485) (width 0.25) (layer "F.Cu") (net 2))
 (segment (start 120.142 91.7956) (end 119.7356 92.202) (width 0.25) (layer "F.Cu") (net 2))
 (segment (start 120.142 90.489) (end 120.142 91.7956) (width 0.25) (layer "F.Cu") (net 2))
 (segment (start 125.0696 88.8492) (end 123.9243 88.8492) (width 0.25) (layer "F.Cu") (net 2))
 (segment (start 109.728 87.282) (end 109.728 89.0016) (width 0.25) (layer "F.Cu") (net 2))
 (via (at 119.7356 86.614) (size 0.508) (drill 0.254) (layers "F.Cu" "B.Cu") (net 2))
 (via (at 109.6772 89.0524) (size 0.508) (drill 0.254) (layers "F.Cu" "B.Cu") (free) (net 2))
 (via (at 119.7356 92.202) (size 0.508) (drill 0.254) (layers "F.Cu" "B.Cu") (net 2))
 (via (at 125.0696 88.8492) (size 0.508) (drill 0.254) (layers "F.Cu" "B.Cu") (free) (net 2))
 (via (at 109.5248 98.298) (size 0.508) (drill 0.254) (layers "F.Cu" "B.Cu") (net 2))
 (segment (start 117.587521 92.508449) (end 120.142 95.062928) (width 0.25) (layer "F.Cu") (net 6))
 (segment (start 109.728 94.057) (end 111.276551 92.508449) (width 0.25) (layer "F.Cu") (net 6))
 (segment (start 120.142 97.346) (end 120.396 97.6) (width 0.25) (layer "F.Cu") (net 6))
 (segment (start 120.142 95.062928) (end 120.142 95.439) (width 0.25) (layer "F.Cu") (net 6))
 (segment (start 120.142 95.439) (end 120.142 97.346) (width 0.25) (layer "F.Cu") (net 6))
 (segment (start 109.728 94.582) (end 109.728 94.057) (width 0.25) (layer "F.Cu") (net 6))
 (segment (start 111.276551 92.508449) (end 117.587521 92.508449) (width 0.25) (layer "F.Cu") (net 6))
 (segment (start 116.332 95.822) (end 114.554 97.6) (width 0.25) (layer "F.Cu") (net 8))
 (segment (start 112.268 94.057) (end 112.917511 93.407489) (width 0.25) (layer "F.Cu") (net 8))
 (segment (start 112.917511 93.407489) (end 114.300489 93.407489) (width 0.25) (layer "F.Cu") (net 8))
 (segment (start 114.300489 93.407489) (end 116.332 95.439) (width 0.25) (layer "F.Cu") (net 8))
 (segment (start 112.268 94.582) (end 112.268 94.057) (width 0.25) (layer "F.Cu") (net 8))
 (segment (start 116.332 95.439) (end 116.332 95.822) (width 0.25) (layer "F.Cu") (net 8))
 (segment (start 110.998 94.582) (end 110.998 94.057) (width 0.25) (layer "F.Cu") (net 7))
 (segment (start 112.097031 92.957969) (end 115.563969 92.957969) (width 0.25) (layer "F.Cu") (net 7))
 (segment (start 110.998 94.057) (end 112.097031 92.957969) (width 0.25) (layer "F.Cu") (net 7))
 (segment (start 118.872 95.439) (end 117.602 95.439) (width 0.25) (layer "F.Cu") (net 7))
 (segment (start 117.602 94.996) (end 117.602 95.439) (width 0.25) (layer "F.Cu") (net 7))
 (segment (start 117.602 95.439) (end 117.602 97.6) (width 0.25) (layer "F.Cu") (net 7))
 (segment (start 115.563969 92.957969) (end 117.602 94.996) (width 0.25) (layer "F.Cu") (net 7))
 (segment (start 129.9972 88.9) (end 132.08 88.9) (width 0.25) (layer "F.Cu") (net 9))
 (segment (start 124.291428 87.0735) (end 124.775 87.0735) (width 0.25) (layer "F.Cu") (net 9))
 (segment (start 128.1684 87.0712) (end 129.9972 88.9) (width 0.25) (layer "F.Cu") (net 9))
 (segment (start 118.872 90.489) (end 118.872 90.112928) (width 0.25) (layer "F.Cu") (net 9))
 (segment (start 120.084928 88.9) (end 122.464928 88.9) (width 0.25) (layer "F.Cu") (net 9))
 (segment (start 124.7773 87.0712) (end 128.1684 87.0712) (width 0.25) (layer "F.Cu") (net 9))
 (segment (start 124.775 87.0735) (end 124.7773 87.0712) (width 0.25) (layer "F.Cu") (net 9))
 (segment (start 122.464928 88.9) (end 124.291428 87.0735) (width 0.25) (layer "F.Cu") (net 9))
 (segment (start 118.872 90.112928) (end 120.084928 88.9) (width 0.25) (layer "F.Cu") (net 9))
 (segment (start 128.354598 86.62168) (end 129.362918 87.63) (width 0.25) (layer "F.Cu") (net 10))
 (segment (start 122.875 87.0735) (end 123.93702 86.01148) (width 0.25) (layer "F.Cu") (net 10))
 (segment (start 125.4246 86.01148) (end 126.0348 86.62168) (width 0.25) (layer "F.Cu") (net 10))
 (segment (start 117.602 90.112928) (end 119.576928 88.138) (width 0.25) (layer "F.Cu") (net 10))
 (segment (start 126.0348 86.62168) (end 128.354598 86.62168) (width 0.25) (layer "F.Cu") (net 10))
 (segment (start 117.602 90.489) (end 117.602 90.112928) (width 0.25) (layer "F.Cu") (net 10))
 (segment (start 129.362918 87.63) (end 132.08 87.63) (width 0.25) (layer "F.Cu") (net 10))
 (segment (start 119.576928 88.138) (end 121.8105 88.138) (width 0.25) (layer "F.Cu") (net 10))
 (segment (start 121.8105 88.138) (end 122.875 87.0735) (width 0.25) (layer "F.Cu") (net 10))
 (segment (start 123.93702 86.01148) (end 125.4246 86.01148) (width 0.25) (layer "F.Cu") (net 10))
 (segment (start 112.268 88.456) (end 106.426 94.298) (width 0.25) (layer "F.Cu") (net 4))
 (segment (start 106.108 93.98) (end 102.616 93.98) (width 0.25) (layer "F.Cu") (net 4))
 (segment (start 112.268 87.282) (end 112.268 88.456) (width 0.25) (layer "F.Cu") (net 4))
 (segment (start 106.426 94.298) (end 106.108 93.98) (width 0.25) (layer "F.Cu") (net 4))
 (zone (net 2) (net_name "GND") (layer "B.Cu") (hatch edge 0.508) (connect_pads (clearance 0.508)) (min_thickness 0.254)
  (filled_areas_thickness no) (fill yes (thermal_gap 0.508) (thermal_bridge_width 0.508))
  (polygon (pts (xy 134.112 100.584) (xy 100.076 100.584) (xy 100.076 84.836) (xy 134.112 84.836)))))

